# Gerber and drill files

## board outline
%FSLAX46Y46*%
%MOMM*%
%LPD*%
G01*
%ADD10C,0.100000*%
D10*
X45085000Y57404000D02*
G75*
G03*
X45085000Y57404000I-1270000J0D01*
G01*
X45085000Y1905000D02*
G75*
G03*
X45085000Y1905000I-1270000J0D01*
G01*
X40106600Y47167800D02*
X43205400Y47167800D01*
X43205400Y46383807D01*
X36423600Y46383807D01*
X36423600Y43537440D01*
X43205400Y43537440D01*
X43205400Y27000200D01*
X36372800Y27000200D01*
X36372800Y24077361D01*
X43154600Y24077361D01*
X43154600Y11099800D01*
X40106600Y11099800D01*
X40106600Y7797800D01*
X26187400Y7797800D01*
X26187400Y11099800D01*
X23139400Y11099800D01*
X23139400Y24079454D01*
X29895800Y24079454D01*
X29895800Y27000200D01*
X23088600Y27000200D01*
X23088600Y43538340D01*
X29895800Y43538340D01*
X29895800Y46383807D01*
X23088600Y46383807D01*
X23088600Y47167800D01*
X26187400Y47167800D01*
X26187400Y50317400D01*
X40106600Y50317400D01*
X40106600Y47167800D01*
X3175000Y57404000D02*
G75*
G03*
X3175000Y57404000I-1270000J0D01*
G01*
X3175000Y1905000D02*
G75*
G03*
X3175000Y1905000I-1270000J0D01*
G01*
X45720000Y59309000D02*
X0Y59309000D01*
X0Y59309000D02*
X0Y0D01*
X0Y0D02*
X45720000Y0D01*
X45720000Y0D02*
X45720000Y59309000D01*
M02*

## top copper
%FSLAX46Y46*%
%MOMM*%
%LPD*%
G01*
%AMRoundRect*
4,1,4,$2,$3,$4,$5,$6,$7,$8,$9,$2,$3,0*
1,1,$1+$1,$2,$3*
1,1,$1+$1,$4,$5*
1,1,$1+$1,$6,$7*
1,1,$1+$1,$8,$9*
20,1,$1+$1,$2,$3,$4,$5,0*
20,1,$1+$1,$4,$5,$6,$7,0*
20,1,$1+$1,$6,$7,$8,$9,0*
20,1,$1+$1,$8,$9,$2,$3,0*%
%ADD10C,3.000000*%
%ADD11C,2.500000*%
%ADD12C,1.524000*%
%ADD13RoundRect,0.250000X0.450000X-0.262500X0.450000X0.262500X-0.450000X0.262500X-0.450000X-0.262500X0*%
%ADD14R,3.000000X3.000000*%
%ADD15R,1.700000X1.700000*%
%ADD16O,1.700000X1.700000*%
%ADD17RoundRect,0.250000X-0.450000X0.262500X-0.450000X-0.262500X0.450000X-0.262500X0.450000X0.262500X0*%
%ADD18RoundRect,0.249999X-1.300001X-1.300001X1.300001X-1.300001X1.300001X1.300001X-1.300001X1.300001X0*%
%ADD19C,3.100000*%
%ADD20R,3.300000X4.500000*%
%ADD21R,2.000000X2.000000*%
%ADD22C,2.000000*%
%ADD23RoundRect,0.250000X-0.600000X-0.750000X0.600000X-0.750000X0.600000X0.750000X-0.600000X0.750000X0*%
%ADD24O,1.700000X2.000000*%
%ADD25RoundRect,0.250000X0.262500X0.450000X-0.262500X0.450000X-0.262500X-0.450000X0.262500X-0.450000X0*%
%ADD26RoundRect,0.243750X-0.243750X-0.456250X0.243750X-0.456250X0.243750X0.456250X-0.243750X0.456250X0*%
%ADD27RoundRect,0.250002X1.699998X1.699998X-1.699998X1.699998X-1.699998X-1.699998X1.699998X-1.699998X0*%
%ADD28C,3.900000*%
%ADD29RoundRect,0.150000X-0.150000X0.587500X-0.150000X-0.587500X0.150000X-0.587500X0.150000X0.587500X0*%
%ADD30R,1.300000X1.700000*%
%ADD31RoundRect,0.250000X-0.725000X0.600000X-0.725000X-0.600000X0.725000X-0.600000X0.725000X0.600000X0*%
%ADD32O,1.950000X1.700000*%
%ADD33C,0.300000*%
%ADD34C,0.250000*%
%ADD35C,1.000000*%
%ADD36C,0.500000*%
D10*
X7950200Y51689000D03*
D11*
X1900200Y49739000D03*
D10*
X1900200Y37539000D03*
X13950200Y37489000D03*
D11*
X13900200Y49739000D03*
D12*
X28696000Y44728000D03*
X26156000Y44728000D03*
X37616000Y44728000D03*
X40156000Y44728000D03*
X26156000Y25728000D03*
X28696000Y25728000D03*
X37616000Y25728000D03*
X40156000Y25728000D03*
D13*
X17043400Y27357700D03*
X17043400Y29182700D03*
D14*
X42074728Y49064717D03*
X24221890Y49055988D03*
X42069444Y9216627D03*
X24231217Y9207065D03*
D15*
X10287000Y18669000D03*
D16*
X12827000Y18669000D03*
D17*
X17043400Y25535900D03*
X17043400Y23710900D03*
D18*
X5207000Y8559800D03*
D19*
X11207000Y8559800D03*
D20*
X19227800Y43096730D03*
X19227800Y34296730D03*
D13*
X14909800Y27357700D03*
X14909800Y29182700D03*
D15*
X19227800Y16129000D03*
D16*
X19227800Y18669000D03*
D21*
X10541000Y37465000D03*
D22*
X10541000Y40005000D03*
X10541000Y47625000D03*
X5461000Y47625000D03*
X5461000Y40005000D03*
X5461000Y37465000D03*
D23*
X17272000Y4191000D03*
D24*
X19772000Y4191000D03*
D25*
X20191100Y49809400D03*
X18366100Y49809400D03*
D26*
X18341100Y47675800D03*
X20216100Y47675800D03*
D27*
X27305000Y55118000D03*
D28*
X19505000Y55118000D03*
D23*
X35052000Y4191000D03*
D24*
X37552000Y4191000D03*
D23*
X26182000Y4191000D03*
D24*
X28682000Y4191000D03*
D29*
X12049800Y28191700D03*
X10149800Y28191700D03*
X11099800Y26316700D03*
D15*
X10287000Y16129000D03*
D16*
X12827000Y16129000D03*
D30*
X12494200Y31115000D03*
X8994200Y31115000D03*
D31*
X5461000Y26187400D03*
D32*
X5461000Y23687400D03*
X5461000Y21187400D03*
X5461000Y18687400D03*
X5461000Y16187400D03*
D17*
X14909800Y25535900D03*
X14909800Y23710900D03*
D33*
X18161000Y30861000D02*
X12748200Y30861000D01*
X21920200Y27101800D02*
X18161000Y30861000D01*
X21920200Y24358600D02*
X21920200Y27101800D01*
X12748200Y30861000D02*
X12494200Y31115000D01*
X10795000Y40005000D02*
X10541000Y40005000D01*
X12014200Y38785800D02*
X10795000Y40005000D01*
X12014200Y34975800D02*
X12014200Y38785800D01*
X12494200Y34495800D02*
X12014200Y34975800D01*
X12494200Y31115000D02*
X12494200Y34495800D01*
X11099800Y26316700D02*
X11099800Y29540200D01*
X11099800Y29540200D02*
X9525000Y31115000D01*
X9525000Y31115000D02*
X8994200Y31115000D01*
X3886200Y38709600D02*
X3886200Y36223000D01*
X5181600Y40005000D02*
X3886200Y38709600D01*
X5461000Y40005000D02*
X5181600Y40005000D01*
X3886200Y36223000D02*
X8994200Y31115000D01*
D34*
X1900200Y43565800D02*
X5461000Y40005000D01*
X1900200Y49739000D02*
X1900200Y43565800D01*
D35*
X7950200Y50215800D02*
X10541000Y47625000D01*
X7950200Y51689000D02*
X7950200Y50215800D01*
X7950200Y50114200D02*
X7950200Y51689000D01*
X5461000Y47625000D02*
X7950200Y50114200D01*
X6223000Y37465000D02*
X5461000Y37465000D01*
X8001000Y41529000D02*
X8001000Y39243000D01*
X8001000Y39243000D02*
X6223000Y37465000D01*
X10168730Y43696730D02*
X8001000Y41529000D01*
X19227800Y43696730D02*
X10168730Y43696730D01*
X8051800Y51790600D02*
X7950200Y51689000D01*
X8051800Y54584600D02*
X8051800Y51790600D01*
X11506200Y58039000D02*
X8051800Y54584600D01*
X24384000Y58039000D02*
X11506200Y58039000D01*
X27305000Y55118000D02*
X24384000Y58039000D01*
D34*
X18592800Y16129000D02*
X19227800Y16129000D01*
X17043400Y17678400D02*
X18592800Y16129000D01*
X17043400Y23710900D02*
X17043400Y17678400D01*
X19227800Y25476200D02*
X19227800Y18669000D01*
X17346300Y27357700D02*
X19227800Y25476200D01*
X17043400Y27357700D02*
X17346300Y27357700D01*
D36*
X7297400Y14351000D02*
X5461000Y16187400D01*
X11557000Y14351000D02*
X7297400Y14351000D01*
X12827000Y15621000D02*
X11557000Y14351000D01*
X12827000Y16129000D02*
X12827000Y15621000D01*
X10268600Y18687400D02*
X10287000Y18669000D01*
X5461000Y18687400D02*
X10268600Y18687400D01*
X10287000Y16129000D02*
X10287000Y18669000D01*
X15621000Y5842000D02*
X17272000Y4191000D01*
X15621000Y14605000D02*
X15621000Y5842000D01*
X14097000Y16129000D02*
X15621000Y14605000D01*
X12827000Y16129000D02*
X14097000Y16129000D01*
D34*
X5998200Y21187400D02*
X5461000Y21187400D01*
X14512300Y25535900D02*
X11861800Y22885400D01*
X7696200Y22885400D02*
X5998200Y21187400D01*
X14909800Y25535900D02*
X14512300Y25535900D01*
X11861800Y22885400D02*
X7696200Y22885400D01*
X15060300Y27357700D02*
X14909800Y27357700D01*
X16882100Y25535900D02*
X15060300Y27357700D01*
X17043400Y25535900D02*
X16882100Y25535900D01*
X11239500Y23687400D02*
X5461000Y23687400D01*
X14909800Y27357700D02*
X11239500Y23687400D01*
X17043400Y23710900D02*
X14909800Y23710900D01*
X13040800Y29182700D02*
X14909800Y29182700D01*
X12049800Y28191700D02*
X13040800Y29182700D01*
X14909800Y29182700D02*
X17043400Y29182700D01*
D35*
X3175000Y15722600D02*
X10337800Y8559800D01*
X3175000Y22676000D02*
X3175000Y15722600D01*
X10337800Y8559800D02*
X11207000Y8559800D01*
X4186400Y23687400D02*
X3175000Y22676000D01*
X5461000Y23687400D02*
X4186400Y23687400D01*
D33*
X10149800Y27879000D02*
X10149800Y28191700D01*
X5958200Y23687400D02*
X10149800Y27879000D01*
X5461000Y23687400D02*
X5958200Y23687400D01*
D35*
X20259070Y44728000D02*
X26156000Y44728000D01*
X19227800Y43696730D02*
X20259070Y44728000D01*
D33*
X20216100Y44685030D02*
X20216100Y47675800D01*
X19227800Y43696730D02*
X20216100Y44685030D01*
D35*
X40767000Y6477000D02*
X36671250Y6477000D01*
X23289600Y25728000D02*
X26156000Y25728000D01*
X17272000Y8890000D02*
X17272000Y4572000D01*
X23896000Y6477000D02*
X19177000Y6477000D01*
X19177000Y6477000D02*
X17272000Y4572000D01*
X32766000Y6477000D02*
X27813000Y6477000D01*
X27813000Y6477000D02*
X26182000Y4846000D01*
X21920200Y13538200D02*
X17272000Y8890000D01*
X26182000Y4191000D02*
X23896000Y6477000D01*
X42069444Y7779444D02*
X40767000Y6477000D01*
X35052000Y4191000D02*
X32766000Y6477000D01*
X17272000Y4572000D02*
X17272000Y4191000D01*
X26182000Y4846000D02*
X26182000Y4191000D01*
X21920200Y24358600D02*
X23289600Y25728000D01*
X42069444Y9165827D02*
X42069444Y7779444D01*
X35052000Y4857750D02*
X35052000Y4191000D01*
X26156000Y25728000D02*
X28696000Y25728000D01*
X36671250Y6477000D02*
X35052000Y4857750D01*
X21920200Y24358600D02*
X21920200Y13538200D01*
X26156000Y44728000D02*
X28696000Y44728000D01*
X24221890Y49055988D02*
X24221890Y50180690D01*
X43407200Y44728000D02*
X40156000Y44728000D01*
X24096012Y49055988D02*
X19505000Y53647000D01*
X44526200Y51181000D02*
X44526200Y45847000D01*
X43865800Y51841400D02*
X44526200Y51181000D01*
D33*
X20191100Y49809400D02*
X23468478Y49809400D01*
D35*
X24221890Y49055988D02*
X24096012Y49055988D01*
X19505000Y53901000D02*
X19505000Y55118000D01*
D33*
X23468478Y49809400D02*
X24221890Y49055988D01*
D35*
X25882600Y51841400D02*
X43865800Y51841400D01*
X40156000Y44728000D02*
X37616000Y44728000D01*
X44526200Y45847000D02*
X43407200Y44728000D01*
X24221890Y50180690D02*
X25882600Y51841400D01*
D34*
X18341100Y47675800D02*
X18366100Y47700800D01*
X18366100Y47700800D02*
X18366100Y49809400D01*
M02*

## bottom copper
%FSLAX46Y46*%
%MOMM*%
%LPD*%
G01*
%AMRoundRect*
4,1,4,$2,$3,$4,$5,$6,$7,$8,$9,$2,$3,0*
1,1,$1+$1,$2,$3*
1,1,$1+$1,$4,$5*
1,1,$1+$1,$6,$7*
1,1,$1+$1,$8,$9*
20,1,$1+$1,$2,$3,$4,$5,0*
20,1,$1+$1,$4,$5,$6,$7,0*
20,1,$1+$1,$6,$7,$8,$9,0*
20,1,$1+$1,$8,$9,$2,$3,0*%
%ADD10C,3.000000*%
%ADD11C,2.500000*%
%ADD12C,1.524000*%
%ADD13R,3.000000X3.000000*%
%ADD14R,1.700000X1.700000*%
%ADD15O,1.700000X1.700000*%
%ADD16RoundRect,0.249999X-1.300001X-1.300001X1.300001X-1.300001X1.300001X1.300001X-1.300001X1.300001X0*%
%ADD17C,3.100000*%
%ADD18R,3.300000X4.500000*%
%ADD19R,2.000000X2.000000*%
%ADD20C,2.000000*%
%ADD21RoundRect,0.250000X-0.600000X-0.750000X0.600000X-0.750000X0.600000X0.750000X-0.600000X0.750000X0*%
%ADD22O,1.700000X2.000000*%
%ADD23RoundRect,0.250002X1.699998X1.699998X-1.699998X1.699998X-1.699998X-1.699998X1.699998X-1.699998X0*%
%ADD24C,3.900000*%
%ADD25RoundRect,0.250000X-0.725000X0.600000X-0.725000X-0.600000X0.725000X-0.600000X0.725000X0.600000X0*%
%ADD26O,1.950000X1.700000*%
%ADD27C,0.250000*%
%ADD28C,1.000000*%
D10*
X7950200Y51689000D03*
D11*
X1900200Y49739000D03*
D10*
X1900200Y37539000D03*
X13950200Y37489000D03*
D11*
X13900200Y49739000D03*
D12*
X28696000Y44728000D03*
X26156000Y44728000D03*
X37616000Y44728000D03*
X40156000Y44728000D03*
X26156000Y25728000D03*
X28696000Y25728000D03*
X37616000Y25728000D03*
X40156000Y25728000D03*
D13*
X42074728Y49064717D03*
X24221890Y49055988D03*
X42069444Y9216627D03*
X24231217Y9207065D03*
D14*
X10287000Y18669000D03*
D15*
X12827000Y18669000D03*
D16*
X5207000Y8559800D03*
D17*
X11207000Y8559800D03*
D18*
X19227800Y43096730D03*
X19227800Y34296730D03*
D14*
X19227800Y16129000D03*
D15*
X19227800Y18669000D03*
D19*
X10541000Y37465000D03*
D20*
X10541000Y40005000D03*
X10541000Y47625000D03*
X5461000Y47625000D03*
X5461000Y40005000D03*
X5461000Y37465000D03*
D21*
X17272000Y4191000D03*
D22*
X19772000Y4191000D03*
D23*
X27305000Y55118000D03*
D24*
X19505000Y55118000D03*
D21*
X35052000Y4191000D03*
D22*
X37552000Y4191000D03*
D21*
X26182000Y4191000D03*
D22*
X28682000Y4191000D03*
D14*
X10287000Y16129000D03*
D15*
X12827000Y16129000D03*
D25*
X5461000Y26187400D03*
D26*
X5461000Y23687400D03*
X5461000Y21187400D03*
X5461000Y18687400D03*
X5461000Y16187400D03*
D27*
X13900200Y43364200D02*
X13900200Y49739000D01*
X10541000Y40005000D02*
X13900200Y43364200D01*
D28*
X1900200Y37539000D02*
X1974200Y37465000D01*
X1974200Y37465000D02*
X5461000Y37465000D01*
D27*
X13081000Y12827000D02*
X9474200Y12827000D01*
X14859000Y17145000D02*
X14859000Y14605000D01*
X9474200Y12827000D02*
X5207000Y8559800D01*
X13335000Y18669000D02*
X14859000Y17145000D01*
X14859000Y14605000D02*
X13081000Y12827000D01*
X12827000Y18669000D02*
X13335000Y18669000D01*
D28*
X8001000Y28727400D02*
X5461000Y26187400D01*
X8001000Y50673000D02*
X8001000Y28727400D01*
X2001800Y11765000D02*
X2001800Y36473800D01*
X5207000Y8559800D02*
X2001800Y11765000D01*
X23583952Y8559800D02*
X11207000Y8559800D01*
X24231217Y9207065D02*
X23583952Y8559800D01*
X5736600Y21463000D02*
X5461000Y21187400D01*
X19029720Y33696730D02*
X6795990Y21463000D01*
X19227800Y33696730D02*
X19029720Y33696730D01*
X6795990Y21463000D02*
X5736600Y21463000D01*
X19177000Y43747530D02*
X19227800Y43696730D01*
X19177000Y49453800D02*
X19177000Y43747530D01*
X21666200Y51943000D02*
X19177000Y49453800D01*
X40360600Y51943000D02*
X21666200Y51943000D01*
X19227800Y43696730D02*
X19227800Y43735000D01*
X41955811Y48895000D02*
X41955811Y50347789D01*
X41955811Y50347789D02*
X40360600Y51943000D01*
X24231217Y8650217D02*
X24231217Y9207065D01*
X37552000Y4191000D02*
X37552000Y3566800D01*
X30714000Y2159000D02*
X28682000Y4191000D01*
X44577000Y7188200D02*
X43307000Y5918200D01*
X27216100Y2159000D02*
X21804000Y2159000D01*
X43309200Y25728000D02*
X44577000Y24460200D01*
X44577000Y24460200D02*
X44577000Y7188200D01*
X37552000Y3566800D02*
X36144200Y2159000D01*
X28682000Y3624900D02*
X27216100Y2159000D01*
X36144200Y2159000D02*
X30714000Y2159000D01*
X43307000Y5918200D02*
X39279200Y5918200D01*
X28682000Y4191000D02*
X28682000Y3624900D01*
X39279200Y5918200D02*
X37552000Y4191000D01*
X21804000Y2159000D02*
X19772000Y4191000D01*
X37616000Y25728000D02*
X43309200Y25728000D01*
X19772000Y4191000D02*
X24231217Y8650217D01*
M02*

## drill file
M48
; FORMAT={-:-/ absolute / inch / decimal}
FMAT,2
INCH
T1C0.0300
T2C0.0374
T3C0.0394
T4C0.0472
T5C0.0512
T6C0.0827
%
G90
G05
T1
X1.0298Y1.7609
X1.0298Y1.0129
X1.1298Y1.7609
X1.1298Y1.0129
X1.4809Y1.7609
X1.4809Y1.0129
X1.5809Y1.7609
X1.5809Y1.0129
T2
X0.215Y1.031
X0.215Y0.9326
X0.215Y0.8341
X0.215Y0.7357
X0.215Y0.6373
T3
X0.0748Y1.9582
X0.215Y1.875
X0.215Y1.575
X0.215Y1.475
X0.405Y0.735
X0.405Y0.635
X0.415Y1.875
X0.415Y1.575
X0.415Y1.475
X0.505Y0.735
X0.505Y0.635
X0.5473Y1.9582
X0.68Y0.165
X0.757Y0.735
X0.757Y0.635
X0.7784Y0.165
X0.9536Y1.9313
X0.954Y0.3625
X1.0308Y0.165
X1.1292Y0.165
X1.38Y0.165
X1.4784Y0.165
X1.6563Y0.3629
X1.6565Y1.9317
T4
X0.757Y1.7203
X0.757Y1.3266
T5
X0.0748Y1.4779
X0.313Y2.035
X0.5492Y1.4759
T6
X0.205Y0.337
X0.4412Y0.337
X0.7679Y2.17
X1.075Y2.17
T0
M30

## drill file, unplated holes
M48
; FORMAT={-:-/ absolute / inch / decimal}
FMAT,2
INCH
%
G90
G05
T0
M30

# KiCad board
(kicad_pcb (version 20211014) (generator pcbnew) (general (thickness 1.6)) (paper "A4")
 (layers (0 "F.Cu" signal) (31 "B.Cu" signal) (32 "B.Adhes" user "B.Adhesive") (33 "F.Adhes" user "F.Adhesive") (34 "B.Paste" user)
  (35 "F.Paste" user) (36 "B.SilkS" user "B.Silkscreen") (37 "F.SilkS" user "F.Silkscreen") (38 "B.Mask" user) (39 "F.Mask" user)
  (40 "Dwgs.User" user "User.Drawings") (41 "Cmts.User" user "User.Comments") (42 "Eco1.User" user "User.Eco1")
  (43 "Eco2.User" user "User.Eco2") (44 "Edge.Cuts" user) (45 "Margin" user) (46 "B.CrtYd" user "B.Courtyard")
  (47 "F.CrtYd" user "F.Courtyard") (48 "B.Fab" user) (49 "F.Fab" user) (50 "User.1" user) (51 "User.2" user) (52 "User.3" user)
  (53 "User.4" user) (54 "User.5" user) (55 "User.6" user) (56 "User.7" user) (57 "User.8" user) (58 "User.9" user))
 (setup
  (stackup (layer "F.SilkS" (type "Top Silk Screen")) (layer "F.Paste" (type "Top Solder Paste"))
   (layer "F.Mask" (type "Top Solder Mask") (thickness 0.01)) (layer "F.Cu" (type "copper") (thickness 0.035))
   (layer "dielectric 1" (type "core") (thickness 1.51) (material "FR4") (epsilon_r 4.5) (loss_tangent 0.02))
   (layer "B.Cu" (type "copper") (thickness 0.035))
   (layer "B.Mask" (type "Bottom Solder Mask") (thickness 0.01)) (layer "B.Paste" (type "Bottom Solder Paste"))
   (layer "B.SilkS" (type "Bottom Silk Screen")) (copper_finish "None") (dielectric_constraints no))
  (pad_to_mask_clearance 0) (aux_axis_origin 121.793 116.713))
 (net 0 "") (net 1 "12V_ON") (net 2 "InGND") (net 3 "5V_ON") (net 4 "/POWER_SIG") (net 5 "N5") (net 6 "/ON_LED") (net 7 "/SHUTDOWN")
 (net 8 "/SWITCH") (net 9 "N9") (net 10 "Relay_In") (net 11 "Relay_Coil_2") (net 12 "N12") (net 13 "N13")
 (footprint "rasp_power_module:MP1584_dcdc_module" (layer "F.Cu") (at 163.449 70.485 -90)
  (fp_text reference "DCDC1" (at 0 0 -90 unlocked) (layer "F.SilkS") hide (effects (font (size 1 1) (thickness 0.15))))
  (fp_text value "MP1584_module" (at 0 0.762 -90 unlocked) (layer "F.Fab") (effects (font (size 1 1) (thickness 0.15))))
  (pad "1" thru_hole circle (at 1.5 12.96 270) (size 1.524 1.524) (drill 0.762) (layers *.Cu *.Mask) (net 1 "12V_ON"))
  (pad "1" thru_hole circle (at 1.5 15.5 270) (size 1.524 1.524) (drill 0.762) (layers *.Cu *.Mask) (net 1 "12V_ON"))
  (pad "2" thru_hole circle (at 1.5 4.04 270) (size 1.524 1.524) (drill 0.762) (layers *.Cu *.Mask) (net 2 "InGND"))
  (pad "2" thru_hole circle (at 1.5 1.5 270) (size 1.524 1.524) (drill 0.762) (layers *.Cu *.Mask) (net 2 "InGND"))
  (pad "3" thru_hole circle (at 20.5 15.5 270) (size 1.524 1.524) (drill 0.762) (layers *.Cu *.Mask) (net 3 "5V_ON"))
  (pad "3" thru_hole circle (at 20.5 12.96 270) (size 1.524 1.524) (drill 0.762) (layers *.Cu *.Mask) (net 3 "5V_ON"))
  (pad "4" thru_hole circle (at 20.5 4.04 270) (size 1.524 1.524) (drill 0.762) (layers *.Cu *.Mask) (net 2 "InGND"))
  (pad "4" thru_hole circle (at 20.5 1.5 270) (size 1.524 1.524) (drill 0.762) (layers *.Cu *.Mask) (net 2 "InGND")))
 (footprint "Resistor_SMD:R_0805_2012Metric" (layer "F.Cu") (at 138.8364 88.4428 90)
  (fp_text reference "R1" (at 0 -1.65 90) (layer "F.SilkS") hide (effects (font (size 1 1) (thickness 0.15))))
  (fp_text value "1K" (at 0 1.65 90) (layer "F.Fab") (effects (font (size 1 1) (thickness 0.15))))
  (pad "1" smd roundrect (at -0.9125 0 90) (size 1.025 1.4) (layers "F.Cu" "F.Paste" "F.Mask") (roundrect_rratio 0.243902439)
   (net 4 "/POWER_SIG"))
  (pad "2" smd roundrect (at 0.9125 0 90) (size 1.025 1.4) (layers "F.Cu" "F.Paste" "F.Mask") (roundrect_rratio 0.243902439) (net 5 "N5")))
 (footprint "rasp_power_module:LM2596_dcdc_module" (layer "F.Cu") (at 154.94 87.5792 -90)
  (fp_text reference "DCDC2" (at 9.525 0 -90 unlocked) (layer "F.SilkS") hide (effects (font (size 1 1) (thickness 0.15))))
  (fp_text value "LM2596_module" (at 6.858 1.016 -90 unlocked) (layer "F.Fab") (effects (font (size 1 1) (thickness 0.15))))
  (pad "1" thru_hole rect (at -19.930917 -8.927728 270) (size 3 3) (drill 1) (layers *.Cu *.Mask) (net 1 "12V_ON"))
  (pad "2" thru_hole rect (at -19.922188 8.92511 270) (size 3 3) (drill 1) (layers *.Cu *.Mask) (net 2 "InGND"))
  (pad "3" thru_hole rect (at 19.917173 -8.922444 270) (size 3 3) (drill 1) (layers *.Cu *.Mask) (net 3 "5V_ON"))
  (pad "4" thru_hole rect (at 19.926735 8.915783 270) (size 3 3) (drill 1) (layers *.Cu *.Mask) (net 2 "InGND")))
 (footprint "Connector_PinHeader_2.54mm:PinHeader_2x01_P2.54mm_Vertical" (layer "F.Cu") (at 132.08 98.044)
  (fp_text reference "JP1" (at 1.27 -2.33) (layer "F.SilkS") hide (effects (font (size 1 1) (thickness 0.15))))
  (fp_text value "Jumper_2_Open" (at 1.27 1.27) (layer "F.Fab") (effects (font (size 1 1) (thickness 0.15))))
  (pad "1" thru_hole rect (at 0 0) (size 1.7 1.7) (drill 1) (layers *.Cu *.Mask) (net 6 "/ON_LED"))
  (pad "2" thru_hole oval (at 2.54 0) (size 1.7 1.7) (drill 1) (layers *.Cu *.Mask) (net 1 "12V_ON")))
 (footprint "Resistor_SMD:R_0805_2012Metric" (layer "F.Cu") (at 138.8364 92.0896 -90)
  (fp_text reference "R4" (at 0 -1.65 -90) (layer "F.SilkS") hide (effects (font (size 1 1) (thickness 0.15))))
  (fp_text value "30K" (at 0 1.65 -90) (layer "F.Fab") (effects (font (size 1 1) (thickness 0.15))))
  (pad "1" smd roundrect (at -0.9125 0 270) (size 1.025 1.4) (layers "F.Cu" "F.Paste" "F.Mask") (roundrect_rratio 0.243902439)
   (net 2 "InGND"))
  (pad "2" smd roundrect (at 0.9125 0 270) (size 1.025 1.4) (layers "F.Cu" "F.Paste" "F.Mask") (roundrect_rratio 0.243902439)
   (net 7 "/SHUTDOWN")))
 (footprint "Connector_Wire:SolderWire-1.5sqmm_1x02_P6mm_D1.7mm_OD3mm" (layer "F.Cu") (at 127 108.1532)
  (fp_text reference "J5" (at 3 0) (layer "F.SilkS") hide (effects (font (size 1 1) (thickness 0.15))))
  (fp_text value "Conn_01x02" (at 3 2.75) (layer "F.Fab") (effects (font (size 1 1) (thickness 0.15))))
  (pad "1" thru_hole roundrect (at 0 0) (size 3.1 3.1) (drill 2.1) (layers *.Cu *.Mask) (roundrect_rratio 0.08064483871) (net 1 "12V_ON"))
  (pad "2" thru_hole circle (at 6 0) (size 3.1 3.1) (drill 2.1) (layers *.Cu *.Mask) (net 2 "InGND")))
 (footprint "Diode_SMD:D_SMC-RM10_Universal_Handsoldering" (layer "F.Cu") (at 141.0208 78.01627 -90)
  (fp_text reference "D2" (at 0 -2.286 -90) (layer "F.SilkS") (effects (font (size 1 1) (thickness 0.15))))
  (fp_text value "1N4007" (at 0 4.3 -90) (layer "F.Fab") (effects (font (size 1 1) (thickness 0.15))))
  (pad "1" thru_hole rect (at -5 0 270) (size 4.5 3.3) (drill 1.2 (offset 0.6 0)) (layers *.Cu *.Mask) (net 1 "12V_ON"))
  (pad "2" thru_hole rect (at 5 0 90) (size 4.5 3.3) (drill 1.2 (offset 0.6 0)) (layers *.Cu *.Mask) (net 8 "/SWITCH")))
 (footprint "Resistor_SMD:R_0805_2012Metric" (layer "F.Cu") (at 136.7028 88.4428 90)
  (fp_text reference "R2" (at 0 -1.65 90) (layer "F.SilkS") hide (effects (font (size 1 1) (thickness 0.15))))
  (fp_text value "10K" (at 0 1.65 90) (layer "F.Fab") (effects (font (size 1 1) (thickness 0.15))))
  (pad "1" smd roundrect (at -0.9125 0 90) (size 1.025 1.4) (layers "F.Cu" "F.Paste" "F.Mask") (roundrect_rratio 0.243902439)
   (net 2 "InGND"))
  (pad "2" smd roundrect (at 0.9125 0 90) (size 1.025 1.4) (layers "F.Cu" "F.Paste" "F.Mask") (roundrect_rratio 0.243902439) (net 5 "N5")))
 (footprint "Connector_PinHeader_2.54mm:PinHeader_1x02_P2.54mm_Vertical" (layer "F.Cu") (at 141.0208 100.584 180)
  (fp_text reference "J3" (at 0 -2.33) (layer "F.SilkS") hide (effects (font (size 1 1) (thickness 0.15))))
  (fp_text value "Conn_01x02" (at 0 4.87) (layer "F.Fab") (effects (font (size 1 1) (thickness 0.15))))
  (pad "1" thru_hole rect (at 0 0 180) (size 1.7 1.7) (drill 1) (layers *.Cu *.Mask) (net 7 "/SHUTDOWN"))
  (pad "2" thru_hole oval (at 0 2.54 180) (size 1.7 1.7) (drill 1) (layers *.Cu *.Mask) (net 4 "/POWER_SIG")))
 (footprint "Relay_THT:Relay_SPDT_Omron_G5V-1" (layer "F.Cu") (at 132.334 79.248 180)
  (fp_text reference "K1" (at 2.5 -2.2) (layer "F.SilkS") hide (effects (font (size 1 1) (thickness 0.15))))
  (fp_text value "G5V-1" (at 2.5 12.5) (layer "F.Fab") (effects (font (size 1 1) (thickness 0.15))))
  (pad "1" thru_hole rect (at 0 0 180) (size 2 2) (drill 1) (layers *.Cu *.Mask) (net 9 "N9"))
  (pad "2" thru_hole circle (at 0 2.54 180) (size 2 2) (drill 1) (layers *.Cu *.Mask) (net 3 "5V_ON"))
  (pad "5" thru_hole circle (at 0 10.16 180) (size 2 2) (drill 1) (layers *.Cu *.Mask) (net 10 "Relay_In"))
  (pad "6" thru_hole circle (at 5.08 10.16 180) (size 2 2) (drill 1) (layers *.Cu *.Mask) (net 10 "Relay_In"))
  (pad "9" thru_hole circle (at 5.08 2.54 180) (size 2 2) (drill 1) (layers *.Cu *.Mask) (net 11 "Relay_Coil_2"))
  (pad "10" thru_hole circle (at 5.08 0 180) (size 2 2) (drill 1) (layers *.Cu *.Mask) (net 1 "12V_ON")))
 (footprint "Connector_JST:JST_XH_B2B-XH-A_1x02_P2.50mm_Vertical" (layer "F.Cu") (at 139.065 112.522)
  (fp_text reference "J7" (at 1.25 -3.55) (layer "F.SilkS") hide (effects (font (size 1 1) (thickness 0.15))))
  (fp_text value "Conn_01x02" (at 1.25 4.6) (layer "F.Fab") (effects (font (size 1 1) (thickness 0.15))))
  (pad "1" thru_hole roundrect (at 0 0) (size 1.7 2) (drill 1) (layers *.Cu *.Mask) (roundrect_rratio 0.1470588235) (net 3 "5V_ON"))
  (pad "2" thru_hole oval (at 2.5 0) (size 1.7 2) (drill 1) (layers *.Cu *.Mask) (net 2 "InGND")))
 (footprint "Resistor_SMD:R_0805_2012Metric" (layer "F.Cu") (at 141.0716 66.9036 180)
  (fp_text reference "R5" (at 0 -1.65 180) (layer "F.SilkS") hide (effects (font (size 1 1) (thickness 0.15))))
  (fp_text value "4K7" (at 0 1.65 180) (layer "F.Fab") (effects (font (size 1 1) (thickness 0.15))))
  (pad "1" smd roundrect (at -0.9125 0 180) (size 1.025 1.4) (layers "F.Cu" "F.Paste" "F.Mask") (roundrect_rratio 0.243902439)
   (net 2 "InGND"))
  (pad "2" smd roundrect (at 0.9125 0 180) (size 1.025 1.4) (layers "F.Cu" "F.Paste" "F.Mask") (roundrect_rratio 0.243902439) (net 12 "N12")))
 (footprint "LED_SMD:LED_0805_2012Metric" (layer "F.Cu") (at 141.0716 69.0372)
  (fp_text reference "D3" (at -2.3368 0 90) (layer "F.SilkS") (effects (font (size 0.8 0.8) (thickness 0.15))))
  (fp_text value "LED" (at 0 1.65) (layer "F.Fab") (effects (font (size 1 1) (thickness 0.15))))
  (pad "1" smd roundrect (at -0.9375 0) (size 0.975 1.4) (layers "F.Cu" "F.Paste" "F.Mask") (roundrect_rratio 0.25) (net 12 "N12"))
  (pad "2" smd roundrect (at 0.9375 0) (size 0.975 1.4) (layers "F.Cu" "F.Paste" "F.Mask") (roundrect_rratio 0.25) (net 1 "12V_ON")))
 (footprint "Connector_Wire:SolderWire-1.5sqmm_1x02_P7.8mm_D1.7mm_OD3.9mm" (layer "F.Cu") (at 149.098 61.595 180)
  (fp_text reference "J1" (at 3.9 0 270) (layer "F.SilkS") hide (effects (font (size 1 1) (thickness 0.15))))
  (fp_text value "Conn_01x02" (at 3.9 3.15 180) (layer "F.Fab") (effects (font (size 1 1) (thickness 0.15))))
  (pad "1" thru_hole roundrect (at 0 0 180) (size 3.9 3.9) (drill 2.1) (layers *.Cu *.Mask) (roundrect_rratio 0.06410307692)
   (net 10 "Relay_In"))
  (pad "2" thru_hole circle (at 7.8 0 180) (size 3.9 3.9) (drill 2.1) (layers *.Cu *.Mask) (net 2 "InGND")))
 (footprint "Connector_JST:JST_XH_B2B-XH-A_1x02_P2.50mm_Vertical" (layer "F.Cu") (at 156.845 112.522)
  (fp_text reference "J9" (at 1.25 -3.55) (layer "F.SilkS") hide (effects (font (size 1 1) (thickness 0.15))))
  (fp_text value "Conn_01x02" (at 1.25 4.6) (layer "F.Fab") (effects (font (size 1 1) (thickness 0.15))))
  (pad "1" thru_hole roundrect (at 0 0) (size 1.7 2) (drill 1) (layers *.Cu *.Mask) (roundrect_rratio 0.1470588235) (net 3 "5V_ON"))
  (pad "2" thru_hole oval (at 2.5 0) (size 1.7 2) (drill 1) (layers *.Cu *.Mask) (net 2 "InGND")))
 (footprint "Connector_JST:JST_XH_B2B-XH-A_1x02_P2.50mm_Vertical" (layer "F.Cu") (at 147.975 112.522)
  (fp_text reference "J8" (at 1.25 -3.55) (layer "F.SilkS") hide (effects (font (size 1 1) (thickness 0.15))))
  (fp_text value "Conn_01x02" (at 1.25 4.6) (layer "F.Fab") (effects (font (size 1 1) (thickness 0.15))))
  (pad "1" thru_hole roundrect (at 0 0) (size 1.7 2) (drill 1) (layers *.Cu *.Mask) (roundrect_rratio 0.1470588235) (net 3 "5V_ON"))
  (pad "2" thru_hole oval (at 2.5 0) (size 1.7 2) (drill 1) (layers *.Cu *.Mask) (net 2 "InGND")))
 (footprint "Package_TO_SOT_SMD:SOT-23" (layer "F.Cu") (at 132.8928 89.4588 -90)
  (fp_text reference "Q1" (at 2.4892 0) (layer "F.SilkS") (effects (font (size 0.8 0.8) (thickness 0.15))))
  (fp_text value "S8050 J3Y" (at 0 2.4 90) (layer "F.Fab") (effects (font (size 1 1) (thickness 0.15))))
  (pad "1" smd roundrect (at -0.9375 -0.95 270) (size 1.475 0.6) (layers "F.Cu" "F.Paste" "F.Mask") (roundrect_rratio 0.25) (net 5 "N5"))
  (pad "2" smd roundrect (at -0.9375 0.95 270) (size 1.475 0.6) (layers "F.Cu" "F.Paste" "F.Mask") (roundrect_rratio 0.25) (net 2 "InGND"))
  (pad "3" smd roundrect (at 0.9375 0 270) (size 1.475 0.6) (layers "F.Cu" "F.Paste" "F.Mask") (roundrect_rratio 0.25)
   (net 11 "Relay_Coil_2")))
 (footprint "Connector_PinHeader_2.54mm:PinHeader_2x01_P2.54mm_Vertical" (layer "F.Cu") (at 132.08 100.584)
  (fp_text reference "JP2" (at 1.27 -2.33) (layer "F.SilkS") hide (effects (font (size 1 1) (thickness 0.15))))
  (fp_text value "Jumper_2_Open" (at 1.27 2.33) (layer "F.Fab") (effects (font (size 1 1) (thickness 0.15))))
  (pad "1" thru_hole rect (at 0 0) (size 1.7 1.7) (drill 1) (layers *.Cu *.Mask) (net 6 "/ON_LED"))
  (pad "2" thru_hole oval (at 2.54 0) (size 1.7 1.7) (drill 1) (layers *.Cu *.Mask) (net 3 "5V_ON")))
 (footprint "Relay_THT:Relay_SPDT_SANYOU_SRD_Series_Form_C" (layer "F.Cu") (at 129.7432 65.024 -90)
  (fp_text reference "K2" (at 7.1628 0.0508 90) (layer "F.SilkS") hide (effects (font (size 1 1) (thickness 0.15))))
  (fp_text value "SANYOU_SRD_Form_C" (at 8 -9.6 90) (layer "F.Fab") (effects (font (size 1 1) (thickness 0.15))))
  (pad "1" thru_hole circle (at 0 0) (size 3 3) (drill 1.3) (layers *.Cu *.Mask) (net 10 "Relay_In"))
  (pad "2" thru_hole circle (at 1.95 6.05) (size 2.5 2.5) (drill 1) (layers *.Cu *.Mask) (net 11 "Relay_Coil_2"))
  (pad "3" thru_hole circle (at 14.15 6.05) (size 3 3) (drill 1.3) (layers *.Cu *.Mask) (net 1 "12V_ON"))
  (pad "4" thru_hole circle (at 14.2 -6) (size 3 3) (drill 1.3) (layers *.Cu *.Mask) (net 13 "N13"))
  (pad "5" thru_hole circle (at 1.95 -5.95) (size 2.5 2.5) (drill 1) (layers *.Cu *.Mask) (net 3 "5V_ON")))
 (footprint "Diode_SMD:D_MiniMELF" (layer "F.Cu") (at 132.5372 85.598 180)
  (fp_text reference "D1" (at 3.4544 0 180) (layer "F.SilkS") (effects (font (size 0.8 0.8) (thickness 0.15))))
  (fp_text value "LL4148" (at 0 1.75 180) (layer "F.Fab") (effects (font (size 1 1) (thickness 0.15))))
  (pad "1" smd rect (at -1.75 0 180) (size 1.3 1.7) (layers "F.Cu" "F.Paste" "F.Mask") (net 3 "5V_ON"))
  (pad "2" smd rect (at 1.75 0 180) (size 1.3 1.7) (layers "F.Cu" "F.Paste" "F.Mask") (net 11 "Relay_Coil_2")))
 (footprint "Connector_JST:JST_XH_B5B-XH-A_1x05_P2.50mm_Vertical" (layer "F.Cu") (at 127.254 90.5256 -90)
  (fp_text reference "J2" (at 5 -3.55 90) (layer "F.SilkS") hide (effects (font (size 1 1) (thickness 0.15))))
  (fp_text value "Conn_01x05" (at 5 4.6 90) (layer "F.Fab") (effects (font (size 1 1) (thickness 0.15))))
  (pad "1" thru_hole roundrect (at 0 0 270) (size 1.7 1.95) (drill 0.95) (layers *.Cu *.Mask) (roundrect_rratio 0.1470588235)
   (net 10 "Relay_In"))
  (pad "2" thru_hole oval (at 2.5 0 270) (size 1.7 1.95) (drill 0.95) (layers *.Cu *.Mask) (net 2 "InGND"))
  (pad "3" thru_hole oval (at 5 0 270) (size 1.7 1.95) (drill 0.95) (layers *.Cu *.Mask) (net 8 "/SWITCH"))
  (pad "4" thru_hole oval (at 7.5 0 270) (size 1.7 1.95) (drill 0.95) (layers *.Cu *.Mask) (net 6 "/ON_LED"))
  (pad "5" thru_hole oval (at 10 0 270) (size 1.7 1.95) (drill 0.95) (layers *.Cu *.Mask) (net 3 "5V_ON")))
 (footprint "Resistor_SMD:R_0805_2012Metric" (layer "F.Cu") (at 136.7028 92.0896 -90)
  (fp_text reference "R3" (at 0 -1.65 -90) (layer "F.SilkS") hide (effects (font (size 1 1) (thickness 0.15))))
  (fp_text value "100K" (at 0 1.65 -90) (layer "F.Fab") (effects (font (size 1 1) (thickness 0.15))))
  (pad "1" smd roundrect (at -0.9125 0 270) (size 1.025 1.4) (layers "F.Cu" "F.Paste" "F.Mask") (roundrect_rratio 0.243902439)
   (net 8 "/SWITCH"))
  (pad "2" smd roundrect (at 0.9125 0 270) (size 1.025 1.4) (layers "F.Cu" "F.Paste" "F.Mask") (roundrect_rratio 0.243902439)
   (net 7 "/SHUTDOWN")))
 (gr_circle (center 165.608 59.309) (end 166.878 59.309) (layer "Edge.Cuts") (width 0.1) (fill none))
 (gr_circle (center 165.608 114.808) (end 166.878 114.808) (layer "Edge.Cuts") (width 0.1) (fill none))
 (gr_poly
  (pts (xy 151.6888 73.17466) (xy 151.6888 70.329193) (xy 144.8816 70.329193) (xy 144.8816 69.5452) (xy 147.9804 69.5452)
   (xy 147.9804 66.3956) (xy 161.8996 66.3956) (xy 161.8996 69.5452) (xy 164.9984 69.5452) (xy 164.9984 70.329193) (xy 158.2166 70.329193)
   (xy 158.2166 73.17556) (xy 164.9984 73.17556) (xy 164.9984 89.7128) (xy 158.1658 89.7128) (xy 158.1658 92.635639) (xy 164.9476 92.635639)
   (xy 164.9476 105.6132) (xy 161.8996 105.6132) (xy 161.8996 108.9152) (xy 147.9804 108.9152) (xy 147.9804 105.6132) (xy 144.9324 105.6132)
   (xy 144.9324 92.633546) (xy 151.6888 92.633546) (xy 151.6888 89.7128) (xy 144.8816 89.7128) (xy 144.8816 73.17466))
  (layer "Edge.Cuts") (width 0.1) (fill none))
 (gr_circle (center 123.698 59.309) (end 124.968 59.309) (layer "Edge.Cuts") (width 0.1) (fill none))
 (gr_circle (center 123.698 114.808) (end 124.968 114.808) (layer "Edge.Cuts") (width 0.1) (fill none))
 (gr_rect (start 167.513 57.404) (end 121.793 116.713) (layer "Edge.Cuts") (width 0.1) (fill none))
 (segment (start 123.6932 66.974) (end 123.6932 73.1472) (width 0.25) (layer "F.Cu") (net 11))
 (segment (start 127.254 76.708) (end 126.9746 76.708) (width 0.3) (layer "F.Cu") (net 11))
 (segment (start 123.6932 73.1472) (end 127.254 76.708) (width 0.25) (layer "F.Cu") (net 11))
 (segment (start 132.8928 87.1728) (end 131.318 85.598) (width 0.3) (layer "F.Cu") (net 11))
 (segment (start 125.6792 80.49) (end 130.7872 85.598) (width 0.3) (layer "F.Cu") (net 11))
 (segment (start 132.8928 90.3963) (end 132.8928 87.1728) (width 0.3) (layer "F.Cu") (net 11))
 (segment (start 126.9746 76.708) (end 125.6792 78.0034) (width 0.3) (layer "F.Cu") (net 11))
 (segment (start 125.6792 78.0034) (end 125.6792 80.49) (width 0.3) (layer "F.Cu") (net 11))
 (segment (start 131.318 85.598) (end 130.7872 85.598) (width 0.3) (layer "F.Cu") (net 11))
 (segment (start 162.56 110.236) (end 158.46425 110.236) (width 1) (layer "F.Cu") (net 3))
 (segment (start 139.954 85.852) (end 134.5412 85.852) (width 0.3) (layer "F.Cu") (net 3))
 (segment (start 145.0826 90.985) (end 147.949 90.985) (width 1) (layer "F.Cu") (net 3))
 (segment (start 139.065 107.823) (end 139.065 112.141) (width 1) (layer "F.Cu") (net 3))
 (segment (start 134.62 100.584) (end 134.62 101.092) (width 0.5) (layer "F.Cu") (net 3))
 (segment (start 145.689 110.236) (end 140.97 110.236) (width 1) (layer "F.Cu") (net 3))
 (segment (start 140.97 110.236) (end 139.065 112.141) (width 1) (layer "F.Cu") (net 3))
 (segment (start 134.2872 82.2172) (end 133.8072 81.7372) (width 0.3) (layer "F.Cu") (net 3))
 (segment (start 154.559 110.236) (end 149.606 110.236) (width 1) (layer "F.Cu") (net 3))
 (segment (start 149.606 110.236) (end 147.975 111.867) (width 1) (layer "F.Cu") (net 3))
 (segment (start 143.7132 103.1748) (end 139.065 107.823) (width 1) (layer "F.Cu") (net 3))
 (segment (start 134.62 101.092) (end 133.35 102.362) (width 0.5) (layer "F.Cu") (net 3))
 (segment (start 133.8072 77.9272) (end 132.588 76.708) (width 0.3) (layer "F.Cu") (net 3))
 (segment (start 147.975 112.522) (end 145.689 110.236) (width 1) (layer "F.Cu") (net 3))
 (segment (start 132.588 76.708) (end 132.334 76.708) (width 0.3) (layer "F.Cu") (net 3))
 (segment (start 135.89 100.584) (end 137.414 102.108) (width 0.5) (layer "F.Cu") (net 3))
 (segment (start 163.862444 108.933556) (end 162.56 110.236) (width 1) (layer "F.Cu") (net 3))
 (segment (start 134.62 100.584) (end 135.89 100.584) (width 0.5) (layer "F.Cu") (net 3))
 (segment (start 143.7132 89.6112) (end 139.954 85.852) (width 0.3) (layer "F.Cu") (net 3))
 (segment (start 129.0904 102.362) (end 127.254 100.5256) (width 0.5) (layer "F.Cu") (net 3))
 (segment (start 137.414 102.108) (end 137.414 110.871) (width 0.5) (layer "F.Cu") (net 3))
 (segment (start 156.845 112.522) (end 154.559 110.236) (width 1) (layer "F.Cu") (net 3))
 (segment (start 139.065 112.141) (end 139.065 112.522) (width 1) (layer "F.Cu") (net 3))
 (segment (start 134.5412 85.852) (end 134.2872 85.598) (width 0.3) (layer "F.Cu") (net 3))
 (segment (start 137.414 110.871) (end 139.065 112.522) (width 0.5) (layer "F.Cu") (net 3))
 (segment (start 133.35 102.362) (end 129.0904 102.362) (width 0.5) (layer "F.Cu") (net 3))
 (segment (start 143.7132 92.3544) (end 143.7132 89.6112) (width 0.3) (layer "F.Cu") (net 3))
 (segment (start 147.975 111.867) (end 147.975 112.522) (width 1) (layer "F.Cu") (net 3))
 (segment (start 134.2872 85.598) (end 134.2872 82.2172) (width 0.3) (layer "F.Cu") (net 3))
 (segment (start 143.7132 92.3544) (end 145.0826 90.985) (width 1) (layer "F.Cu") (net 3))
 (segment (start 163.862444 107.547173) (end 163.862444 108.933556) (width 1) (layer "F.Cu") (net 3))
 (segment (start 133.8072 81.7372) (end 133.8072 77.9272) (width 0.3) (layer "F.Cu") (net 3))
 (segment (start 156.845 111.85525) (end 156.845 112.522) (width 1) (layer "F.Cu") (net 3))
 (segment (start 147.949 90.985) (end 150.489 90.985) (width 1) (layer "F.Cu") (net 3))
 (segment (start 158.46425 110.236) (end 156.845 111.85525) (width 1) (layer "F.Cu") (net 3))
 (segment (start 143.7132 92.3544) (end 143.7132 103.1748) (width 1) (layer "F.Cu") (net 3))
 (segment (start 135.6932 73.3488) (end 135.6932 66.974) (width 0.25) (layer "B.Cu") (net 3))
 (segment (start 132.334 76.708) (end 135.6932 73.3488) (width 0.25) (layer "B.Cu") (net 3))
 (segment (start 142.05207 71.985) (end 147.949 71.985) (width 1) (layer "F.Cu") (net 1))
 (segment (start 141.0208 73.01627) (end 131.96173 73.01627) (width 1) (layer "F.Cu") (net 1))
 (segment (start 142.0091 72.02797) (end 142.0091 69.0372) (width 0.3) (layer "F.Cu") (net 1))
 (segment (start 129.794 77.47) (end 128.016 79.248) (width 1) (layer "F.Cu") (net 1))
 (segment (start 131.96173 73.01627) (end 129.794 75.184) (width 1) (layer "F.Cu") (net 1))
 (segment (start 141.0208 73.01627) (end 142.0091 72.02797) (width 0.3) (layer "F.Cu") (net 1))
 (segment (start 147.949 71.985) (end 150.489 71.985) (width 1) (layer "F.Cu") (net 1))
 (segment (start 141.0208 73.01627) (end 142.05207 71.985) (width 1) (layer "F.Cu") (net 1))
 (segment (start 128.016 79.248) (end 127.254 79.248) (width 1) (layer "F.Cu") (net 1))
 (segment (start 129.794 75.184) (end 129.794 77.47) (width 1) (layer "F.Cu") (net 1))
 (segment (start 123.6932 79.174) (end 123.7672 79.248) (width 1) (layer "B.Cu") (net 1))
 (segment (start 162.1536 64.77) (end 143.4592 64.77) (width 1) (layer "B.Cu") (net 1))
 (segment (start 123.7672 79.248) (end 127.254 79.248) (width 1) (layer "B.Cu") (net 1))
 (segment (start 123.7948 104.948) (end 123.7948 80.2392) (width 1) (layer "B.Cu") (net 1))
 (segment (start 136.652 99.568) (end 136.652 102.108) (width 0.25) (layer "B.Cu") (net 1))
 (segment (start 163.748811 67.818) (end 163.748811 66.365211) (width 1) (layer "B.Cu") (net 1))
 (segment (start 141.0208 73.01627) (end 141.0208 72.978) (width 1) (layer "B.Cu") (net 1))
 (segment (start 134.874 103.886) (end 131.2672 103.886) (width 0.25) (layer "B.Cu") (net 1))
 (segment (start 163.748811 66.365211) (end 162.1536 64.77) (width 1) (layer "B.Cu") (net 1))
 (segment (start 140.97 67.2592) (end 140.97 72.96547) (width 1) (layer "B.Cu") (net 1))
 (segment (start 143.4592 64.77) (end 140.97 67.2592) (width 1) (layer "B.Cu") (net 1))
 (segment (start 134.62 98.044) (end 135.128 98.044) (width 0.25) (layer "B.Cu") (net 1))
 (segment (start 136.652 102.108) (end 134.874 103.886) (width 0.25) (layer "B.Cu") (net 1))
 (segment (start 131.2672 103.886) (end 127 108.1532) (width 0.25) (layer "B.Cu") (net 1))
 (segment (start 135.128 98.044) (end 136.652 99.568) (width 0.25) (layer "B.Cu") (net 1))
 (segment (start 140.97 72.96547) (end 141.0208 73.01627) (width 1) (layer "B.Cu") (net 1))
 (segment (start 127 108.1532) (end 123.7948 104.948) (width 1) (layer "B.Cu") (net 1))
 (segment (start 146.01489 67.657012) (end 146.01489 66.53231) (width 1) (layer "F.Cu") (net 2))
 (segment (start 124.968 100.9904) (end 132.1308 108.1532) (width 1) (layer "F.Cu") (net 2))
 (segment (start 165.2002 71.985) (end 161.949 71.985) (width 1) (layer "F.Cu") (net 2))
 (segment (start 127.254 93.0256) (end 127.7512 93.0256) (width 0.3) (layer "F.Cu") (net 2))
 (segment (start 127.254 93.0256) (end 125.9794 93.0256) (width 1) (layer "F.Cu") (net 2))
 (segment (start 145.889012 67.657012) (end 141.298 63.066) (width 1) (layer "F.Cu") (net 2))
 (segment (start 166.3192 65.532) (end 166.3192 70.866) (width 1) (layer "F.Cu") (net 2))
 (segment (start 165.6588 64.8716) (end 166.3192 65.532) (width 1) (layer "F.Cu") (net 2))
 (segment (start 141.9841 66.9036) (end 145.261478 66.9036) (width 0.3) (layer "F.Cu") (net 2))
 (segment (start 146.01489 67.657012) (end 145.889012 67.657012) (width 1) (layer "F.Cu") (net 2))
 (segment (start 136.7028 89.3553) (end 133.0325 93.0256) (width 0.25) (layer "F.Cu") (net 2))
 (segment (start 138.6751 91.1771) (end 136.8533 89.3553) (width 0.25) (layer "F.Cu") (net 2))
 (segment (start 141.298 62.812) (end 141.298 61.595) (width 1) (layer "F.Cu") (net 2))
 (segment (start 131.9428 88.834) (end 131.9428 88.5213) (width 0.3) (layer "F.Cu") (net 2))
 (segment (start 127.7512 93.0256) (end 131.9428 88.834) (width 0.3) (layer "F.Cu") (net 2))
 (segment (start 133.0325 93.0256) (end 127.254 93.0256) (width 0.25) (layer "F.Cu") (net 2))
 (segment (start 145.261478 66.9036) (end 146.01489 67.657012) (width 0.3) (layer "F.Cu") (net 2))
 (segment (start 147.6756 64.8716) (end 165.6588 64.8716) (width 1) (layer "F.Cu") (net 2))
 (segment (start 132.1308 108.1532) (end 133 108.1532) (width 1) (layer "F.Cu") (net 2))
 (segment (start 161.949 71.985) (end 159.409 71.985) (width 1) (layer "F.Cu") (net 2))
 (segment (start 166.3192 70.866) (end 165.2002 71.985) (width 1) (layer "F.Cu") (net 2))
 (segment (start 146.01489 66.53231) (end 147.6756 64.8716) (width 1) (layer "F.Cu") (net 2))
 (segment (start 125.9794 93.0256) (end 124.968 94.037) (width 1) (layer "F.Cu") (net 2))
 (segment (start 124.968 94.037) (end 124.968 100.9904) (width 1) (layer "F.Cu") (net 2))
 (segment (start 136.8533 89.3553) (end 136.7028 89.3553) (width 0.25) (layer "F.Cu") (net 2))
 (segment (start 138.8364 91.1771) (end 138.6751 91.1771) (width 0.25) (layer "F.Cu") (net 2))
 (segment (start 146.024217 108.062783) (end 146.024217 107.505935) (width 1) (layer "B.Cu") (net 2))
 (segment (start 159.345 112.522) (end 159.345 113.1462) (width 1) (layer "B.Cu") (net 2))
 (segment (start 152.507 114.554) (end 150.475 112.522) (width 1) (layer "B.Cu") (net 2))
 (segment (start 145.376952 108.1532) (end 133 108.1532) (width 1) (layer "B.Cu") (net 2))
 (segment (start 166.37 109.5248) (end 165.1 110.7948) (width 1) (layer "B.Cu") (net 2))
 (segment (start 149.0091 114.554) (end 143.597 114.554) (width 1) (layer "B.Cu") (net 2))
 (segment (start 165.1022 90.985) (end 166.37 92.2528) (width 1) (layer "B.Cu") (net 2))
 (segment (start 166.37 92.2528) (end 166.37 109.5248) (width 1) (layer "B.Cu") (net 2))
 (segment (start 159.345 113.1462) (end 157.9372 114.554) (width 1) (layer "B.Cu") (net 2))
 (segment (start 150.475 113.0881) (end 149.0091 114.554) (width 1) (layer "B.Cu") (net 2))
 (segment (start 157.9372 114.554) (end 152.507 114.554) (width 1) (layer "B.Cu") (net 2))
 (segment (start 146.024217 107.505935) (end 145.376952 108.1532) (width 1) (layer "B.Cu") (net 2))
 (segment (start 165.1 110.7948) (end 161.0722 110.7948) (width 1) (layer "B.Cu") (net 2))
 (segment (start 150.475 112.522) (end 150.475 113.0881) (width 1) (layer "B.Cu") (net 2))
 (segment (start 161.0722 110.7948) (end 159.345 112.522) (width 1) (layer "B.Cu") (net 2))
 (segment (start 143.597 114.554) (end 141.565 112.522) (width 1) (layer "B.Cu") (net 2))
 (segment (start 159.409 90.985) (end 165.1022 90.985) (width 1) (layer "B.Cu") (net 2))
 (segment (start 141.565 112.522) (end 146.024217 108.062783) (width 1) (layer "B.Cu") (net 2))
 (segment (start 136.3053 91.1771) (end 133.6548 93.8276) (width 0.25) (layer "F.Cu") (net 8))
 (segment (start 127.7912 95.5256) (end 127.254 95.5256) (width 0.25) (layer "F.Cu") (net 8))
 (segment (start 136.7028 91.1771) (end 136.3053 91.1771) (width 0.25) (layer "F.Cu") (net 8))
 (segment (start 129.4892 93.8276) (end 127.7912 95.5256) (width 0.25) (layer "F.Cu") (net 8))
 (segment (start 133.6548 93.8276) (end 129.4892 93.8276) (width 0.25) (layer "F.Cu") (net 8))
 (segment (start 141.0208 83.01627) (end 140.82272 83.01627) (width 1) (layer "B.Cu") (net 8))
 (segment (start 140.82272 83.01627) (end 128.58899 95.25) (width 1) (layer "B.Cu") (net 8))
 (segment (start 127.5296 95.25) (end 127.254 95.5256) (width 1) (layer "B.Cu") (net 8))
 (segment (start 128.58899 95.25) (end 127.5296 95.25) (width 1) (layer "B.Cu") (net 8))
 (segment (start 140.1341 69.0372) (end 140.1591 69.0122) (width 0.25) (layer "F.Cu") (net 12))
 (segment (start 140.1591 69.0122) (end 140.1591 66.9036) (width 0.25) (layer "F.Cu") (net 12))
 (segment (start 127.254 98.0256) (end 132.0616 98.0256) (width 0.5) (layer "F.Cu") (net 6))
 (segment (start 132.0616 98.0256) (end 132.08 98.044) (width 0.5) (layer "F.Cu") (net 6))
 (segment (start 132.08 100.584) (end 132.08 98.044) (width 0.5) (layer "F.Cu") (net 6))
 (segment (start 141.0208 91.2368) (end 141.0208 98.044) (width 0.25) (layer "F.Cu") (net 4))
 (segment (start 139.1393 89.3553) (end 141.0208 91.2368) (width 0.25) (layer "F.Cu") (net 4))
 (segment (start 138.8364 89.3553) (end 139.1393 89.3553) (width 0.25) (layer "F.Cu") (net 4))
 (segment (start 138.8364 93.0021) (end 136.7028 93.0021) (width 0.25) (layer "F.Cu") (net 7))
 (segment (start 138.8364 99.0346) (end 140.3858 100.584) (width 0.25) (layer "F.Cu") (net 7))
 (segment (start 138.8364 93.0021) (end 138.8364 99.0346) (width 0.25) (layer "F.Cu") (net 7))
 (segment (start 140.3858 100.584) (end 141.0208 100.584) (width 0.25) (layer "F.Cu") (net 7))
 (segment (start 133.2992 58.674) (end 129.8448 62.1284) (width 1) (layer "F.Cu") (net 10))
 (segment (start 146.177 58.674) (end 133.2992 58.674) (width 1) (layer "F.Cu") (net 10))
 (segment (start 127.254 69.088) (end 129.7432 66.5988) (width 1) (layer "F.Cu") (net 10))
 (segment (start 149.098 61.595) (end 146.177 58.674) (width 1) (layer "F.Cu") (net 10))
 (segment (start 129.7432 66.4972) (end 132.334 69.088) (width 1) (layer "F.Cu") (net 10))
 (segment (start 129.8448 64.9224) (end 129.7432 65.024) (width 1) (layer "F.Cu") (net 10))
 (segment (start 129.7432 66.5988) (end 129.7432 65.024) (width 1) (layer "F.Cu") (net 10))
 (segment (start 129.8448 62.1284) (end 129.8448 64.9224) (width 1) (layer "F.Cu") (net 10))
 (segment (start 129.7432 65.024) (end 129.7432 66.4972) (width 1) (layer "F.Cu") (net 10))
 (segment (start 129.794 66.04) (end 129.794 87.9856) (width 1) (layer "B.Cu") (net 10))
 (segment (start 129.794 87.9856) (end 127.254 90.5256) (width 1) (layer "B.Cu") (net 10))
 (segment (start 134.8338 87.5303) (end 136.7028 87.5303) (width 0.25) (layer "F.Cu") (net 5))
 (segment (start 136.7028 87.5303) (end 138.8364 87.5303) (width 0.25) (layer "F.Cu") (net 5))
 (segment (start 133.8428 88.5213) (end 134.8338 87.5303) (width 0.25) (layer "F.Cu") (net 5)))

